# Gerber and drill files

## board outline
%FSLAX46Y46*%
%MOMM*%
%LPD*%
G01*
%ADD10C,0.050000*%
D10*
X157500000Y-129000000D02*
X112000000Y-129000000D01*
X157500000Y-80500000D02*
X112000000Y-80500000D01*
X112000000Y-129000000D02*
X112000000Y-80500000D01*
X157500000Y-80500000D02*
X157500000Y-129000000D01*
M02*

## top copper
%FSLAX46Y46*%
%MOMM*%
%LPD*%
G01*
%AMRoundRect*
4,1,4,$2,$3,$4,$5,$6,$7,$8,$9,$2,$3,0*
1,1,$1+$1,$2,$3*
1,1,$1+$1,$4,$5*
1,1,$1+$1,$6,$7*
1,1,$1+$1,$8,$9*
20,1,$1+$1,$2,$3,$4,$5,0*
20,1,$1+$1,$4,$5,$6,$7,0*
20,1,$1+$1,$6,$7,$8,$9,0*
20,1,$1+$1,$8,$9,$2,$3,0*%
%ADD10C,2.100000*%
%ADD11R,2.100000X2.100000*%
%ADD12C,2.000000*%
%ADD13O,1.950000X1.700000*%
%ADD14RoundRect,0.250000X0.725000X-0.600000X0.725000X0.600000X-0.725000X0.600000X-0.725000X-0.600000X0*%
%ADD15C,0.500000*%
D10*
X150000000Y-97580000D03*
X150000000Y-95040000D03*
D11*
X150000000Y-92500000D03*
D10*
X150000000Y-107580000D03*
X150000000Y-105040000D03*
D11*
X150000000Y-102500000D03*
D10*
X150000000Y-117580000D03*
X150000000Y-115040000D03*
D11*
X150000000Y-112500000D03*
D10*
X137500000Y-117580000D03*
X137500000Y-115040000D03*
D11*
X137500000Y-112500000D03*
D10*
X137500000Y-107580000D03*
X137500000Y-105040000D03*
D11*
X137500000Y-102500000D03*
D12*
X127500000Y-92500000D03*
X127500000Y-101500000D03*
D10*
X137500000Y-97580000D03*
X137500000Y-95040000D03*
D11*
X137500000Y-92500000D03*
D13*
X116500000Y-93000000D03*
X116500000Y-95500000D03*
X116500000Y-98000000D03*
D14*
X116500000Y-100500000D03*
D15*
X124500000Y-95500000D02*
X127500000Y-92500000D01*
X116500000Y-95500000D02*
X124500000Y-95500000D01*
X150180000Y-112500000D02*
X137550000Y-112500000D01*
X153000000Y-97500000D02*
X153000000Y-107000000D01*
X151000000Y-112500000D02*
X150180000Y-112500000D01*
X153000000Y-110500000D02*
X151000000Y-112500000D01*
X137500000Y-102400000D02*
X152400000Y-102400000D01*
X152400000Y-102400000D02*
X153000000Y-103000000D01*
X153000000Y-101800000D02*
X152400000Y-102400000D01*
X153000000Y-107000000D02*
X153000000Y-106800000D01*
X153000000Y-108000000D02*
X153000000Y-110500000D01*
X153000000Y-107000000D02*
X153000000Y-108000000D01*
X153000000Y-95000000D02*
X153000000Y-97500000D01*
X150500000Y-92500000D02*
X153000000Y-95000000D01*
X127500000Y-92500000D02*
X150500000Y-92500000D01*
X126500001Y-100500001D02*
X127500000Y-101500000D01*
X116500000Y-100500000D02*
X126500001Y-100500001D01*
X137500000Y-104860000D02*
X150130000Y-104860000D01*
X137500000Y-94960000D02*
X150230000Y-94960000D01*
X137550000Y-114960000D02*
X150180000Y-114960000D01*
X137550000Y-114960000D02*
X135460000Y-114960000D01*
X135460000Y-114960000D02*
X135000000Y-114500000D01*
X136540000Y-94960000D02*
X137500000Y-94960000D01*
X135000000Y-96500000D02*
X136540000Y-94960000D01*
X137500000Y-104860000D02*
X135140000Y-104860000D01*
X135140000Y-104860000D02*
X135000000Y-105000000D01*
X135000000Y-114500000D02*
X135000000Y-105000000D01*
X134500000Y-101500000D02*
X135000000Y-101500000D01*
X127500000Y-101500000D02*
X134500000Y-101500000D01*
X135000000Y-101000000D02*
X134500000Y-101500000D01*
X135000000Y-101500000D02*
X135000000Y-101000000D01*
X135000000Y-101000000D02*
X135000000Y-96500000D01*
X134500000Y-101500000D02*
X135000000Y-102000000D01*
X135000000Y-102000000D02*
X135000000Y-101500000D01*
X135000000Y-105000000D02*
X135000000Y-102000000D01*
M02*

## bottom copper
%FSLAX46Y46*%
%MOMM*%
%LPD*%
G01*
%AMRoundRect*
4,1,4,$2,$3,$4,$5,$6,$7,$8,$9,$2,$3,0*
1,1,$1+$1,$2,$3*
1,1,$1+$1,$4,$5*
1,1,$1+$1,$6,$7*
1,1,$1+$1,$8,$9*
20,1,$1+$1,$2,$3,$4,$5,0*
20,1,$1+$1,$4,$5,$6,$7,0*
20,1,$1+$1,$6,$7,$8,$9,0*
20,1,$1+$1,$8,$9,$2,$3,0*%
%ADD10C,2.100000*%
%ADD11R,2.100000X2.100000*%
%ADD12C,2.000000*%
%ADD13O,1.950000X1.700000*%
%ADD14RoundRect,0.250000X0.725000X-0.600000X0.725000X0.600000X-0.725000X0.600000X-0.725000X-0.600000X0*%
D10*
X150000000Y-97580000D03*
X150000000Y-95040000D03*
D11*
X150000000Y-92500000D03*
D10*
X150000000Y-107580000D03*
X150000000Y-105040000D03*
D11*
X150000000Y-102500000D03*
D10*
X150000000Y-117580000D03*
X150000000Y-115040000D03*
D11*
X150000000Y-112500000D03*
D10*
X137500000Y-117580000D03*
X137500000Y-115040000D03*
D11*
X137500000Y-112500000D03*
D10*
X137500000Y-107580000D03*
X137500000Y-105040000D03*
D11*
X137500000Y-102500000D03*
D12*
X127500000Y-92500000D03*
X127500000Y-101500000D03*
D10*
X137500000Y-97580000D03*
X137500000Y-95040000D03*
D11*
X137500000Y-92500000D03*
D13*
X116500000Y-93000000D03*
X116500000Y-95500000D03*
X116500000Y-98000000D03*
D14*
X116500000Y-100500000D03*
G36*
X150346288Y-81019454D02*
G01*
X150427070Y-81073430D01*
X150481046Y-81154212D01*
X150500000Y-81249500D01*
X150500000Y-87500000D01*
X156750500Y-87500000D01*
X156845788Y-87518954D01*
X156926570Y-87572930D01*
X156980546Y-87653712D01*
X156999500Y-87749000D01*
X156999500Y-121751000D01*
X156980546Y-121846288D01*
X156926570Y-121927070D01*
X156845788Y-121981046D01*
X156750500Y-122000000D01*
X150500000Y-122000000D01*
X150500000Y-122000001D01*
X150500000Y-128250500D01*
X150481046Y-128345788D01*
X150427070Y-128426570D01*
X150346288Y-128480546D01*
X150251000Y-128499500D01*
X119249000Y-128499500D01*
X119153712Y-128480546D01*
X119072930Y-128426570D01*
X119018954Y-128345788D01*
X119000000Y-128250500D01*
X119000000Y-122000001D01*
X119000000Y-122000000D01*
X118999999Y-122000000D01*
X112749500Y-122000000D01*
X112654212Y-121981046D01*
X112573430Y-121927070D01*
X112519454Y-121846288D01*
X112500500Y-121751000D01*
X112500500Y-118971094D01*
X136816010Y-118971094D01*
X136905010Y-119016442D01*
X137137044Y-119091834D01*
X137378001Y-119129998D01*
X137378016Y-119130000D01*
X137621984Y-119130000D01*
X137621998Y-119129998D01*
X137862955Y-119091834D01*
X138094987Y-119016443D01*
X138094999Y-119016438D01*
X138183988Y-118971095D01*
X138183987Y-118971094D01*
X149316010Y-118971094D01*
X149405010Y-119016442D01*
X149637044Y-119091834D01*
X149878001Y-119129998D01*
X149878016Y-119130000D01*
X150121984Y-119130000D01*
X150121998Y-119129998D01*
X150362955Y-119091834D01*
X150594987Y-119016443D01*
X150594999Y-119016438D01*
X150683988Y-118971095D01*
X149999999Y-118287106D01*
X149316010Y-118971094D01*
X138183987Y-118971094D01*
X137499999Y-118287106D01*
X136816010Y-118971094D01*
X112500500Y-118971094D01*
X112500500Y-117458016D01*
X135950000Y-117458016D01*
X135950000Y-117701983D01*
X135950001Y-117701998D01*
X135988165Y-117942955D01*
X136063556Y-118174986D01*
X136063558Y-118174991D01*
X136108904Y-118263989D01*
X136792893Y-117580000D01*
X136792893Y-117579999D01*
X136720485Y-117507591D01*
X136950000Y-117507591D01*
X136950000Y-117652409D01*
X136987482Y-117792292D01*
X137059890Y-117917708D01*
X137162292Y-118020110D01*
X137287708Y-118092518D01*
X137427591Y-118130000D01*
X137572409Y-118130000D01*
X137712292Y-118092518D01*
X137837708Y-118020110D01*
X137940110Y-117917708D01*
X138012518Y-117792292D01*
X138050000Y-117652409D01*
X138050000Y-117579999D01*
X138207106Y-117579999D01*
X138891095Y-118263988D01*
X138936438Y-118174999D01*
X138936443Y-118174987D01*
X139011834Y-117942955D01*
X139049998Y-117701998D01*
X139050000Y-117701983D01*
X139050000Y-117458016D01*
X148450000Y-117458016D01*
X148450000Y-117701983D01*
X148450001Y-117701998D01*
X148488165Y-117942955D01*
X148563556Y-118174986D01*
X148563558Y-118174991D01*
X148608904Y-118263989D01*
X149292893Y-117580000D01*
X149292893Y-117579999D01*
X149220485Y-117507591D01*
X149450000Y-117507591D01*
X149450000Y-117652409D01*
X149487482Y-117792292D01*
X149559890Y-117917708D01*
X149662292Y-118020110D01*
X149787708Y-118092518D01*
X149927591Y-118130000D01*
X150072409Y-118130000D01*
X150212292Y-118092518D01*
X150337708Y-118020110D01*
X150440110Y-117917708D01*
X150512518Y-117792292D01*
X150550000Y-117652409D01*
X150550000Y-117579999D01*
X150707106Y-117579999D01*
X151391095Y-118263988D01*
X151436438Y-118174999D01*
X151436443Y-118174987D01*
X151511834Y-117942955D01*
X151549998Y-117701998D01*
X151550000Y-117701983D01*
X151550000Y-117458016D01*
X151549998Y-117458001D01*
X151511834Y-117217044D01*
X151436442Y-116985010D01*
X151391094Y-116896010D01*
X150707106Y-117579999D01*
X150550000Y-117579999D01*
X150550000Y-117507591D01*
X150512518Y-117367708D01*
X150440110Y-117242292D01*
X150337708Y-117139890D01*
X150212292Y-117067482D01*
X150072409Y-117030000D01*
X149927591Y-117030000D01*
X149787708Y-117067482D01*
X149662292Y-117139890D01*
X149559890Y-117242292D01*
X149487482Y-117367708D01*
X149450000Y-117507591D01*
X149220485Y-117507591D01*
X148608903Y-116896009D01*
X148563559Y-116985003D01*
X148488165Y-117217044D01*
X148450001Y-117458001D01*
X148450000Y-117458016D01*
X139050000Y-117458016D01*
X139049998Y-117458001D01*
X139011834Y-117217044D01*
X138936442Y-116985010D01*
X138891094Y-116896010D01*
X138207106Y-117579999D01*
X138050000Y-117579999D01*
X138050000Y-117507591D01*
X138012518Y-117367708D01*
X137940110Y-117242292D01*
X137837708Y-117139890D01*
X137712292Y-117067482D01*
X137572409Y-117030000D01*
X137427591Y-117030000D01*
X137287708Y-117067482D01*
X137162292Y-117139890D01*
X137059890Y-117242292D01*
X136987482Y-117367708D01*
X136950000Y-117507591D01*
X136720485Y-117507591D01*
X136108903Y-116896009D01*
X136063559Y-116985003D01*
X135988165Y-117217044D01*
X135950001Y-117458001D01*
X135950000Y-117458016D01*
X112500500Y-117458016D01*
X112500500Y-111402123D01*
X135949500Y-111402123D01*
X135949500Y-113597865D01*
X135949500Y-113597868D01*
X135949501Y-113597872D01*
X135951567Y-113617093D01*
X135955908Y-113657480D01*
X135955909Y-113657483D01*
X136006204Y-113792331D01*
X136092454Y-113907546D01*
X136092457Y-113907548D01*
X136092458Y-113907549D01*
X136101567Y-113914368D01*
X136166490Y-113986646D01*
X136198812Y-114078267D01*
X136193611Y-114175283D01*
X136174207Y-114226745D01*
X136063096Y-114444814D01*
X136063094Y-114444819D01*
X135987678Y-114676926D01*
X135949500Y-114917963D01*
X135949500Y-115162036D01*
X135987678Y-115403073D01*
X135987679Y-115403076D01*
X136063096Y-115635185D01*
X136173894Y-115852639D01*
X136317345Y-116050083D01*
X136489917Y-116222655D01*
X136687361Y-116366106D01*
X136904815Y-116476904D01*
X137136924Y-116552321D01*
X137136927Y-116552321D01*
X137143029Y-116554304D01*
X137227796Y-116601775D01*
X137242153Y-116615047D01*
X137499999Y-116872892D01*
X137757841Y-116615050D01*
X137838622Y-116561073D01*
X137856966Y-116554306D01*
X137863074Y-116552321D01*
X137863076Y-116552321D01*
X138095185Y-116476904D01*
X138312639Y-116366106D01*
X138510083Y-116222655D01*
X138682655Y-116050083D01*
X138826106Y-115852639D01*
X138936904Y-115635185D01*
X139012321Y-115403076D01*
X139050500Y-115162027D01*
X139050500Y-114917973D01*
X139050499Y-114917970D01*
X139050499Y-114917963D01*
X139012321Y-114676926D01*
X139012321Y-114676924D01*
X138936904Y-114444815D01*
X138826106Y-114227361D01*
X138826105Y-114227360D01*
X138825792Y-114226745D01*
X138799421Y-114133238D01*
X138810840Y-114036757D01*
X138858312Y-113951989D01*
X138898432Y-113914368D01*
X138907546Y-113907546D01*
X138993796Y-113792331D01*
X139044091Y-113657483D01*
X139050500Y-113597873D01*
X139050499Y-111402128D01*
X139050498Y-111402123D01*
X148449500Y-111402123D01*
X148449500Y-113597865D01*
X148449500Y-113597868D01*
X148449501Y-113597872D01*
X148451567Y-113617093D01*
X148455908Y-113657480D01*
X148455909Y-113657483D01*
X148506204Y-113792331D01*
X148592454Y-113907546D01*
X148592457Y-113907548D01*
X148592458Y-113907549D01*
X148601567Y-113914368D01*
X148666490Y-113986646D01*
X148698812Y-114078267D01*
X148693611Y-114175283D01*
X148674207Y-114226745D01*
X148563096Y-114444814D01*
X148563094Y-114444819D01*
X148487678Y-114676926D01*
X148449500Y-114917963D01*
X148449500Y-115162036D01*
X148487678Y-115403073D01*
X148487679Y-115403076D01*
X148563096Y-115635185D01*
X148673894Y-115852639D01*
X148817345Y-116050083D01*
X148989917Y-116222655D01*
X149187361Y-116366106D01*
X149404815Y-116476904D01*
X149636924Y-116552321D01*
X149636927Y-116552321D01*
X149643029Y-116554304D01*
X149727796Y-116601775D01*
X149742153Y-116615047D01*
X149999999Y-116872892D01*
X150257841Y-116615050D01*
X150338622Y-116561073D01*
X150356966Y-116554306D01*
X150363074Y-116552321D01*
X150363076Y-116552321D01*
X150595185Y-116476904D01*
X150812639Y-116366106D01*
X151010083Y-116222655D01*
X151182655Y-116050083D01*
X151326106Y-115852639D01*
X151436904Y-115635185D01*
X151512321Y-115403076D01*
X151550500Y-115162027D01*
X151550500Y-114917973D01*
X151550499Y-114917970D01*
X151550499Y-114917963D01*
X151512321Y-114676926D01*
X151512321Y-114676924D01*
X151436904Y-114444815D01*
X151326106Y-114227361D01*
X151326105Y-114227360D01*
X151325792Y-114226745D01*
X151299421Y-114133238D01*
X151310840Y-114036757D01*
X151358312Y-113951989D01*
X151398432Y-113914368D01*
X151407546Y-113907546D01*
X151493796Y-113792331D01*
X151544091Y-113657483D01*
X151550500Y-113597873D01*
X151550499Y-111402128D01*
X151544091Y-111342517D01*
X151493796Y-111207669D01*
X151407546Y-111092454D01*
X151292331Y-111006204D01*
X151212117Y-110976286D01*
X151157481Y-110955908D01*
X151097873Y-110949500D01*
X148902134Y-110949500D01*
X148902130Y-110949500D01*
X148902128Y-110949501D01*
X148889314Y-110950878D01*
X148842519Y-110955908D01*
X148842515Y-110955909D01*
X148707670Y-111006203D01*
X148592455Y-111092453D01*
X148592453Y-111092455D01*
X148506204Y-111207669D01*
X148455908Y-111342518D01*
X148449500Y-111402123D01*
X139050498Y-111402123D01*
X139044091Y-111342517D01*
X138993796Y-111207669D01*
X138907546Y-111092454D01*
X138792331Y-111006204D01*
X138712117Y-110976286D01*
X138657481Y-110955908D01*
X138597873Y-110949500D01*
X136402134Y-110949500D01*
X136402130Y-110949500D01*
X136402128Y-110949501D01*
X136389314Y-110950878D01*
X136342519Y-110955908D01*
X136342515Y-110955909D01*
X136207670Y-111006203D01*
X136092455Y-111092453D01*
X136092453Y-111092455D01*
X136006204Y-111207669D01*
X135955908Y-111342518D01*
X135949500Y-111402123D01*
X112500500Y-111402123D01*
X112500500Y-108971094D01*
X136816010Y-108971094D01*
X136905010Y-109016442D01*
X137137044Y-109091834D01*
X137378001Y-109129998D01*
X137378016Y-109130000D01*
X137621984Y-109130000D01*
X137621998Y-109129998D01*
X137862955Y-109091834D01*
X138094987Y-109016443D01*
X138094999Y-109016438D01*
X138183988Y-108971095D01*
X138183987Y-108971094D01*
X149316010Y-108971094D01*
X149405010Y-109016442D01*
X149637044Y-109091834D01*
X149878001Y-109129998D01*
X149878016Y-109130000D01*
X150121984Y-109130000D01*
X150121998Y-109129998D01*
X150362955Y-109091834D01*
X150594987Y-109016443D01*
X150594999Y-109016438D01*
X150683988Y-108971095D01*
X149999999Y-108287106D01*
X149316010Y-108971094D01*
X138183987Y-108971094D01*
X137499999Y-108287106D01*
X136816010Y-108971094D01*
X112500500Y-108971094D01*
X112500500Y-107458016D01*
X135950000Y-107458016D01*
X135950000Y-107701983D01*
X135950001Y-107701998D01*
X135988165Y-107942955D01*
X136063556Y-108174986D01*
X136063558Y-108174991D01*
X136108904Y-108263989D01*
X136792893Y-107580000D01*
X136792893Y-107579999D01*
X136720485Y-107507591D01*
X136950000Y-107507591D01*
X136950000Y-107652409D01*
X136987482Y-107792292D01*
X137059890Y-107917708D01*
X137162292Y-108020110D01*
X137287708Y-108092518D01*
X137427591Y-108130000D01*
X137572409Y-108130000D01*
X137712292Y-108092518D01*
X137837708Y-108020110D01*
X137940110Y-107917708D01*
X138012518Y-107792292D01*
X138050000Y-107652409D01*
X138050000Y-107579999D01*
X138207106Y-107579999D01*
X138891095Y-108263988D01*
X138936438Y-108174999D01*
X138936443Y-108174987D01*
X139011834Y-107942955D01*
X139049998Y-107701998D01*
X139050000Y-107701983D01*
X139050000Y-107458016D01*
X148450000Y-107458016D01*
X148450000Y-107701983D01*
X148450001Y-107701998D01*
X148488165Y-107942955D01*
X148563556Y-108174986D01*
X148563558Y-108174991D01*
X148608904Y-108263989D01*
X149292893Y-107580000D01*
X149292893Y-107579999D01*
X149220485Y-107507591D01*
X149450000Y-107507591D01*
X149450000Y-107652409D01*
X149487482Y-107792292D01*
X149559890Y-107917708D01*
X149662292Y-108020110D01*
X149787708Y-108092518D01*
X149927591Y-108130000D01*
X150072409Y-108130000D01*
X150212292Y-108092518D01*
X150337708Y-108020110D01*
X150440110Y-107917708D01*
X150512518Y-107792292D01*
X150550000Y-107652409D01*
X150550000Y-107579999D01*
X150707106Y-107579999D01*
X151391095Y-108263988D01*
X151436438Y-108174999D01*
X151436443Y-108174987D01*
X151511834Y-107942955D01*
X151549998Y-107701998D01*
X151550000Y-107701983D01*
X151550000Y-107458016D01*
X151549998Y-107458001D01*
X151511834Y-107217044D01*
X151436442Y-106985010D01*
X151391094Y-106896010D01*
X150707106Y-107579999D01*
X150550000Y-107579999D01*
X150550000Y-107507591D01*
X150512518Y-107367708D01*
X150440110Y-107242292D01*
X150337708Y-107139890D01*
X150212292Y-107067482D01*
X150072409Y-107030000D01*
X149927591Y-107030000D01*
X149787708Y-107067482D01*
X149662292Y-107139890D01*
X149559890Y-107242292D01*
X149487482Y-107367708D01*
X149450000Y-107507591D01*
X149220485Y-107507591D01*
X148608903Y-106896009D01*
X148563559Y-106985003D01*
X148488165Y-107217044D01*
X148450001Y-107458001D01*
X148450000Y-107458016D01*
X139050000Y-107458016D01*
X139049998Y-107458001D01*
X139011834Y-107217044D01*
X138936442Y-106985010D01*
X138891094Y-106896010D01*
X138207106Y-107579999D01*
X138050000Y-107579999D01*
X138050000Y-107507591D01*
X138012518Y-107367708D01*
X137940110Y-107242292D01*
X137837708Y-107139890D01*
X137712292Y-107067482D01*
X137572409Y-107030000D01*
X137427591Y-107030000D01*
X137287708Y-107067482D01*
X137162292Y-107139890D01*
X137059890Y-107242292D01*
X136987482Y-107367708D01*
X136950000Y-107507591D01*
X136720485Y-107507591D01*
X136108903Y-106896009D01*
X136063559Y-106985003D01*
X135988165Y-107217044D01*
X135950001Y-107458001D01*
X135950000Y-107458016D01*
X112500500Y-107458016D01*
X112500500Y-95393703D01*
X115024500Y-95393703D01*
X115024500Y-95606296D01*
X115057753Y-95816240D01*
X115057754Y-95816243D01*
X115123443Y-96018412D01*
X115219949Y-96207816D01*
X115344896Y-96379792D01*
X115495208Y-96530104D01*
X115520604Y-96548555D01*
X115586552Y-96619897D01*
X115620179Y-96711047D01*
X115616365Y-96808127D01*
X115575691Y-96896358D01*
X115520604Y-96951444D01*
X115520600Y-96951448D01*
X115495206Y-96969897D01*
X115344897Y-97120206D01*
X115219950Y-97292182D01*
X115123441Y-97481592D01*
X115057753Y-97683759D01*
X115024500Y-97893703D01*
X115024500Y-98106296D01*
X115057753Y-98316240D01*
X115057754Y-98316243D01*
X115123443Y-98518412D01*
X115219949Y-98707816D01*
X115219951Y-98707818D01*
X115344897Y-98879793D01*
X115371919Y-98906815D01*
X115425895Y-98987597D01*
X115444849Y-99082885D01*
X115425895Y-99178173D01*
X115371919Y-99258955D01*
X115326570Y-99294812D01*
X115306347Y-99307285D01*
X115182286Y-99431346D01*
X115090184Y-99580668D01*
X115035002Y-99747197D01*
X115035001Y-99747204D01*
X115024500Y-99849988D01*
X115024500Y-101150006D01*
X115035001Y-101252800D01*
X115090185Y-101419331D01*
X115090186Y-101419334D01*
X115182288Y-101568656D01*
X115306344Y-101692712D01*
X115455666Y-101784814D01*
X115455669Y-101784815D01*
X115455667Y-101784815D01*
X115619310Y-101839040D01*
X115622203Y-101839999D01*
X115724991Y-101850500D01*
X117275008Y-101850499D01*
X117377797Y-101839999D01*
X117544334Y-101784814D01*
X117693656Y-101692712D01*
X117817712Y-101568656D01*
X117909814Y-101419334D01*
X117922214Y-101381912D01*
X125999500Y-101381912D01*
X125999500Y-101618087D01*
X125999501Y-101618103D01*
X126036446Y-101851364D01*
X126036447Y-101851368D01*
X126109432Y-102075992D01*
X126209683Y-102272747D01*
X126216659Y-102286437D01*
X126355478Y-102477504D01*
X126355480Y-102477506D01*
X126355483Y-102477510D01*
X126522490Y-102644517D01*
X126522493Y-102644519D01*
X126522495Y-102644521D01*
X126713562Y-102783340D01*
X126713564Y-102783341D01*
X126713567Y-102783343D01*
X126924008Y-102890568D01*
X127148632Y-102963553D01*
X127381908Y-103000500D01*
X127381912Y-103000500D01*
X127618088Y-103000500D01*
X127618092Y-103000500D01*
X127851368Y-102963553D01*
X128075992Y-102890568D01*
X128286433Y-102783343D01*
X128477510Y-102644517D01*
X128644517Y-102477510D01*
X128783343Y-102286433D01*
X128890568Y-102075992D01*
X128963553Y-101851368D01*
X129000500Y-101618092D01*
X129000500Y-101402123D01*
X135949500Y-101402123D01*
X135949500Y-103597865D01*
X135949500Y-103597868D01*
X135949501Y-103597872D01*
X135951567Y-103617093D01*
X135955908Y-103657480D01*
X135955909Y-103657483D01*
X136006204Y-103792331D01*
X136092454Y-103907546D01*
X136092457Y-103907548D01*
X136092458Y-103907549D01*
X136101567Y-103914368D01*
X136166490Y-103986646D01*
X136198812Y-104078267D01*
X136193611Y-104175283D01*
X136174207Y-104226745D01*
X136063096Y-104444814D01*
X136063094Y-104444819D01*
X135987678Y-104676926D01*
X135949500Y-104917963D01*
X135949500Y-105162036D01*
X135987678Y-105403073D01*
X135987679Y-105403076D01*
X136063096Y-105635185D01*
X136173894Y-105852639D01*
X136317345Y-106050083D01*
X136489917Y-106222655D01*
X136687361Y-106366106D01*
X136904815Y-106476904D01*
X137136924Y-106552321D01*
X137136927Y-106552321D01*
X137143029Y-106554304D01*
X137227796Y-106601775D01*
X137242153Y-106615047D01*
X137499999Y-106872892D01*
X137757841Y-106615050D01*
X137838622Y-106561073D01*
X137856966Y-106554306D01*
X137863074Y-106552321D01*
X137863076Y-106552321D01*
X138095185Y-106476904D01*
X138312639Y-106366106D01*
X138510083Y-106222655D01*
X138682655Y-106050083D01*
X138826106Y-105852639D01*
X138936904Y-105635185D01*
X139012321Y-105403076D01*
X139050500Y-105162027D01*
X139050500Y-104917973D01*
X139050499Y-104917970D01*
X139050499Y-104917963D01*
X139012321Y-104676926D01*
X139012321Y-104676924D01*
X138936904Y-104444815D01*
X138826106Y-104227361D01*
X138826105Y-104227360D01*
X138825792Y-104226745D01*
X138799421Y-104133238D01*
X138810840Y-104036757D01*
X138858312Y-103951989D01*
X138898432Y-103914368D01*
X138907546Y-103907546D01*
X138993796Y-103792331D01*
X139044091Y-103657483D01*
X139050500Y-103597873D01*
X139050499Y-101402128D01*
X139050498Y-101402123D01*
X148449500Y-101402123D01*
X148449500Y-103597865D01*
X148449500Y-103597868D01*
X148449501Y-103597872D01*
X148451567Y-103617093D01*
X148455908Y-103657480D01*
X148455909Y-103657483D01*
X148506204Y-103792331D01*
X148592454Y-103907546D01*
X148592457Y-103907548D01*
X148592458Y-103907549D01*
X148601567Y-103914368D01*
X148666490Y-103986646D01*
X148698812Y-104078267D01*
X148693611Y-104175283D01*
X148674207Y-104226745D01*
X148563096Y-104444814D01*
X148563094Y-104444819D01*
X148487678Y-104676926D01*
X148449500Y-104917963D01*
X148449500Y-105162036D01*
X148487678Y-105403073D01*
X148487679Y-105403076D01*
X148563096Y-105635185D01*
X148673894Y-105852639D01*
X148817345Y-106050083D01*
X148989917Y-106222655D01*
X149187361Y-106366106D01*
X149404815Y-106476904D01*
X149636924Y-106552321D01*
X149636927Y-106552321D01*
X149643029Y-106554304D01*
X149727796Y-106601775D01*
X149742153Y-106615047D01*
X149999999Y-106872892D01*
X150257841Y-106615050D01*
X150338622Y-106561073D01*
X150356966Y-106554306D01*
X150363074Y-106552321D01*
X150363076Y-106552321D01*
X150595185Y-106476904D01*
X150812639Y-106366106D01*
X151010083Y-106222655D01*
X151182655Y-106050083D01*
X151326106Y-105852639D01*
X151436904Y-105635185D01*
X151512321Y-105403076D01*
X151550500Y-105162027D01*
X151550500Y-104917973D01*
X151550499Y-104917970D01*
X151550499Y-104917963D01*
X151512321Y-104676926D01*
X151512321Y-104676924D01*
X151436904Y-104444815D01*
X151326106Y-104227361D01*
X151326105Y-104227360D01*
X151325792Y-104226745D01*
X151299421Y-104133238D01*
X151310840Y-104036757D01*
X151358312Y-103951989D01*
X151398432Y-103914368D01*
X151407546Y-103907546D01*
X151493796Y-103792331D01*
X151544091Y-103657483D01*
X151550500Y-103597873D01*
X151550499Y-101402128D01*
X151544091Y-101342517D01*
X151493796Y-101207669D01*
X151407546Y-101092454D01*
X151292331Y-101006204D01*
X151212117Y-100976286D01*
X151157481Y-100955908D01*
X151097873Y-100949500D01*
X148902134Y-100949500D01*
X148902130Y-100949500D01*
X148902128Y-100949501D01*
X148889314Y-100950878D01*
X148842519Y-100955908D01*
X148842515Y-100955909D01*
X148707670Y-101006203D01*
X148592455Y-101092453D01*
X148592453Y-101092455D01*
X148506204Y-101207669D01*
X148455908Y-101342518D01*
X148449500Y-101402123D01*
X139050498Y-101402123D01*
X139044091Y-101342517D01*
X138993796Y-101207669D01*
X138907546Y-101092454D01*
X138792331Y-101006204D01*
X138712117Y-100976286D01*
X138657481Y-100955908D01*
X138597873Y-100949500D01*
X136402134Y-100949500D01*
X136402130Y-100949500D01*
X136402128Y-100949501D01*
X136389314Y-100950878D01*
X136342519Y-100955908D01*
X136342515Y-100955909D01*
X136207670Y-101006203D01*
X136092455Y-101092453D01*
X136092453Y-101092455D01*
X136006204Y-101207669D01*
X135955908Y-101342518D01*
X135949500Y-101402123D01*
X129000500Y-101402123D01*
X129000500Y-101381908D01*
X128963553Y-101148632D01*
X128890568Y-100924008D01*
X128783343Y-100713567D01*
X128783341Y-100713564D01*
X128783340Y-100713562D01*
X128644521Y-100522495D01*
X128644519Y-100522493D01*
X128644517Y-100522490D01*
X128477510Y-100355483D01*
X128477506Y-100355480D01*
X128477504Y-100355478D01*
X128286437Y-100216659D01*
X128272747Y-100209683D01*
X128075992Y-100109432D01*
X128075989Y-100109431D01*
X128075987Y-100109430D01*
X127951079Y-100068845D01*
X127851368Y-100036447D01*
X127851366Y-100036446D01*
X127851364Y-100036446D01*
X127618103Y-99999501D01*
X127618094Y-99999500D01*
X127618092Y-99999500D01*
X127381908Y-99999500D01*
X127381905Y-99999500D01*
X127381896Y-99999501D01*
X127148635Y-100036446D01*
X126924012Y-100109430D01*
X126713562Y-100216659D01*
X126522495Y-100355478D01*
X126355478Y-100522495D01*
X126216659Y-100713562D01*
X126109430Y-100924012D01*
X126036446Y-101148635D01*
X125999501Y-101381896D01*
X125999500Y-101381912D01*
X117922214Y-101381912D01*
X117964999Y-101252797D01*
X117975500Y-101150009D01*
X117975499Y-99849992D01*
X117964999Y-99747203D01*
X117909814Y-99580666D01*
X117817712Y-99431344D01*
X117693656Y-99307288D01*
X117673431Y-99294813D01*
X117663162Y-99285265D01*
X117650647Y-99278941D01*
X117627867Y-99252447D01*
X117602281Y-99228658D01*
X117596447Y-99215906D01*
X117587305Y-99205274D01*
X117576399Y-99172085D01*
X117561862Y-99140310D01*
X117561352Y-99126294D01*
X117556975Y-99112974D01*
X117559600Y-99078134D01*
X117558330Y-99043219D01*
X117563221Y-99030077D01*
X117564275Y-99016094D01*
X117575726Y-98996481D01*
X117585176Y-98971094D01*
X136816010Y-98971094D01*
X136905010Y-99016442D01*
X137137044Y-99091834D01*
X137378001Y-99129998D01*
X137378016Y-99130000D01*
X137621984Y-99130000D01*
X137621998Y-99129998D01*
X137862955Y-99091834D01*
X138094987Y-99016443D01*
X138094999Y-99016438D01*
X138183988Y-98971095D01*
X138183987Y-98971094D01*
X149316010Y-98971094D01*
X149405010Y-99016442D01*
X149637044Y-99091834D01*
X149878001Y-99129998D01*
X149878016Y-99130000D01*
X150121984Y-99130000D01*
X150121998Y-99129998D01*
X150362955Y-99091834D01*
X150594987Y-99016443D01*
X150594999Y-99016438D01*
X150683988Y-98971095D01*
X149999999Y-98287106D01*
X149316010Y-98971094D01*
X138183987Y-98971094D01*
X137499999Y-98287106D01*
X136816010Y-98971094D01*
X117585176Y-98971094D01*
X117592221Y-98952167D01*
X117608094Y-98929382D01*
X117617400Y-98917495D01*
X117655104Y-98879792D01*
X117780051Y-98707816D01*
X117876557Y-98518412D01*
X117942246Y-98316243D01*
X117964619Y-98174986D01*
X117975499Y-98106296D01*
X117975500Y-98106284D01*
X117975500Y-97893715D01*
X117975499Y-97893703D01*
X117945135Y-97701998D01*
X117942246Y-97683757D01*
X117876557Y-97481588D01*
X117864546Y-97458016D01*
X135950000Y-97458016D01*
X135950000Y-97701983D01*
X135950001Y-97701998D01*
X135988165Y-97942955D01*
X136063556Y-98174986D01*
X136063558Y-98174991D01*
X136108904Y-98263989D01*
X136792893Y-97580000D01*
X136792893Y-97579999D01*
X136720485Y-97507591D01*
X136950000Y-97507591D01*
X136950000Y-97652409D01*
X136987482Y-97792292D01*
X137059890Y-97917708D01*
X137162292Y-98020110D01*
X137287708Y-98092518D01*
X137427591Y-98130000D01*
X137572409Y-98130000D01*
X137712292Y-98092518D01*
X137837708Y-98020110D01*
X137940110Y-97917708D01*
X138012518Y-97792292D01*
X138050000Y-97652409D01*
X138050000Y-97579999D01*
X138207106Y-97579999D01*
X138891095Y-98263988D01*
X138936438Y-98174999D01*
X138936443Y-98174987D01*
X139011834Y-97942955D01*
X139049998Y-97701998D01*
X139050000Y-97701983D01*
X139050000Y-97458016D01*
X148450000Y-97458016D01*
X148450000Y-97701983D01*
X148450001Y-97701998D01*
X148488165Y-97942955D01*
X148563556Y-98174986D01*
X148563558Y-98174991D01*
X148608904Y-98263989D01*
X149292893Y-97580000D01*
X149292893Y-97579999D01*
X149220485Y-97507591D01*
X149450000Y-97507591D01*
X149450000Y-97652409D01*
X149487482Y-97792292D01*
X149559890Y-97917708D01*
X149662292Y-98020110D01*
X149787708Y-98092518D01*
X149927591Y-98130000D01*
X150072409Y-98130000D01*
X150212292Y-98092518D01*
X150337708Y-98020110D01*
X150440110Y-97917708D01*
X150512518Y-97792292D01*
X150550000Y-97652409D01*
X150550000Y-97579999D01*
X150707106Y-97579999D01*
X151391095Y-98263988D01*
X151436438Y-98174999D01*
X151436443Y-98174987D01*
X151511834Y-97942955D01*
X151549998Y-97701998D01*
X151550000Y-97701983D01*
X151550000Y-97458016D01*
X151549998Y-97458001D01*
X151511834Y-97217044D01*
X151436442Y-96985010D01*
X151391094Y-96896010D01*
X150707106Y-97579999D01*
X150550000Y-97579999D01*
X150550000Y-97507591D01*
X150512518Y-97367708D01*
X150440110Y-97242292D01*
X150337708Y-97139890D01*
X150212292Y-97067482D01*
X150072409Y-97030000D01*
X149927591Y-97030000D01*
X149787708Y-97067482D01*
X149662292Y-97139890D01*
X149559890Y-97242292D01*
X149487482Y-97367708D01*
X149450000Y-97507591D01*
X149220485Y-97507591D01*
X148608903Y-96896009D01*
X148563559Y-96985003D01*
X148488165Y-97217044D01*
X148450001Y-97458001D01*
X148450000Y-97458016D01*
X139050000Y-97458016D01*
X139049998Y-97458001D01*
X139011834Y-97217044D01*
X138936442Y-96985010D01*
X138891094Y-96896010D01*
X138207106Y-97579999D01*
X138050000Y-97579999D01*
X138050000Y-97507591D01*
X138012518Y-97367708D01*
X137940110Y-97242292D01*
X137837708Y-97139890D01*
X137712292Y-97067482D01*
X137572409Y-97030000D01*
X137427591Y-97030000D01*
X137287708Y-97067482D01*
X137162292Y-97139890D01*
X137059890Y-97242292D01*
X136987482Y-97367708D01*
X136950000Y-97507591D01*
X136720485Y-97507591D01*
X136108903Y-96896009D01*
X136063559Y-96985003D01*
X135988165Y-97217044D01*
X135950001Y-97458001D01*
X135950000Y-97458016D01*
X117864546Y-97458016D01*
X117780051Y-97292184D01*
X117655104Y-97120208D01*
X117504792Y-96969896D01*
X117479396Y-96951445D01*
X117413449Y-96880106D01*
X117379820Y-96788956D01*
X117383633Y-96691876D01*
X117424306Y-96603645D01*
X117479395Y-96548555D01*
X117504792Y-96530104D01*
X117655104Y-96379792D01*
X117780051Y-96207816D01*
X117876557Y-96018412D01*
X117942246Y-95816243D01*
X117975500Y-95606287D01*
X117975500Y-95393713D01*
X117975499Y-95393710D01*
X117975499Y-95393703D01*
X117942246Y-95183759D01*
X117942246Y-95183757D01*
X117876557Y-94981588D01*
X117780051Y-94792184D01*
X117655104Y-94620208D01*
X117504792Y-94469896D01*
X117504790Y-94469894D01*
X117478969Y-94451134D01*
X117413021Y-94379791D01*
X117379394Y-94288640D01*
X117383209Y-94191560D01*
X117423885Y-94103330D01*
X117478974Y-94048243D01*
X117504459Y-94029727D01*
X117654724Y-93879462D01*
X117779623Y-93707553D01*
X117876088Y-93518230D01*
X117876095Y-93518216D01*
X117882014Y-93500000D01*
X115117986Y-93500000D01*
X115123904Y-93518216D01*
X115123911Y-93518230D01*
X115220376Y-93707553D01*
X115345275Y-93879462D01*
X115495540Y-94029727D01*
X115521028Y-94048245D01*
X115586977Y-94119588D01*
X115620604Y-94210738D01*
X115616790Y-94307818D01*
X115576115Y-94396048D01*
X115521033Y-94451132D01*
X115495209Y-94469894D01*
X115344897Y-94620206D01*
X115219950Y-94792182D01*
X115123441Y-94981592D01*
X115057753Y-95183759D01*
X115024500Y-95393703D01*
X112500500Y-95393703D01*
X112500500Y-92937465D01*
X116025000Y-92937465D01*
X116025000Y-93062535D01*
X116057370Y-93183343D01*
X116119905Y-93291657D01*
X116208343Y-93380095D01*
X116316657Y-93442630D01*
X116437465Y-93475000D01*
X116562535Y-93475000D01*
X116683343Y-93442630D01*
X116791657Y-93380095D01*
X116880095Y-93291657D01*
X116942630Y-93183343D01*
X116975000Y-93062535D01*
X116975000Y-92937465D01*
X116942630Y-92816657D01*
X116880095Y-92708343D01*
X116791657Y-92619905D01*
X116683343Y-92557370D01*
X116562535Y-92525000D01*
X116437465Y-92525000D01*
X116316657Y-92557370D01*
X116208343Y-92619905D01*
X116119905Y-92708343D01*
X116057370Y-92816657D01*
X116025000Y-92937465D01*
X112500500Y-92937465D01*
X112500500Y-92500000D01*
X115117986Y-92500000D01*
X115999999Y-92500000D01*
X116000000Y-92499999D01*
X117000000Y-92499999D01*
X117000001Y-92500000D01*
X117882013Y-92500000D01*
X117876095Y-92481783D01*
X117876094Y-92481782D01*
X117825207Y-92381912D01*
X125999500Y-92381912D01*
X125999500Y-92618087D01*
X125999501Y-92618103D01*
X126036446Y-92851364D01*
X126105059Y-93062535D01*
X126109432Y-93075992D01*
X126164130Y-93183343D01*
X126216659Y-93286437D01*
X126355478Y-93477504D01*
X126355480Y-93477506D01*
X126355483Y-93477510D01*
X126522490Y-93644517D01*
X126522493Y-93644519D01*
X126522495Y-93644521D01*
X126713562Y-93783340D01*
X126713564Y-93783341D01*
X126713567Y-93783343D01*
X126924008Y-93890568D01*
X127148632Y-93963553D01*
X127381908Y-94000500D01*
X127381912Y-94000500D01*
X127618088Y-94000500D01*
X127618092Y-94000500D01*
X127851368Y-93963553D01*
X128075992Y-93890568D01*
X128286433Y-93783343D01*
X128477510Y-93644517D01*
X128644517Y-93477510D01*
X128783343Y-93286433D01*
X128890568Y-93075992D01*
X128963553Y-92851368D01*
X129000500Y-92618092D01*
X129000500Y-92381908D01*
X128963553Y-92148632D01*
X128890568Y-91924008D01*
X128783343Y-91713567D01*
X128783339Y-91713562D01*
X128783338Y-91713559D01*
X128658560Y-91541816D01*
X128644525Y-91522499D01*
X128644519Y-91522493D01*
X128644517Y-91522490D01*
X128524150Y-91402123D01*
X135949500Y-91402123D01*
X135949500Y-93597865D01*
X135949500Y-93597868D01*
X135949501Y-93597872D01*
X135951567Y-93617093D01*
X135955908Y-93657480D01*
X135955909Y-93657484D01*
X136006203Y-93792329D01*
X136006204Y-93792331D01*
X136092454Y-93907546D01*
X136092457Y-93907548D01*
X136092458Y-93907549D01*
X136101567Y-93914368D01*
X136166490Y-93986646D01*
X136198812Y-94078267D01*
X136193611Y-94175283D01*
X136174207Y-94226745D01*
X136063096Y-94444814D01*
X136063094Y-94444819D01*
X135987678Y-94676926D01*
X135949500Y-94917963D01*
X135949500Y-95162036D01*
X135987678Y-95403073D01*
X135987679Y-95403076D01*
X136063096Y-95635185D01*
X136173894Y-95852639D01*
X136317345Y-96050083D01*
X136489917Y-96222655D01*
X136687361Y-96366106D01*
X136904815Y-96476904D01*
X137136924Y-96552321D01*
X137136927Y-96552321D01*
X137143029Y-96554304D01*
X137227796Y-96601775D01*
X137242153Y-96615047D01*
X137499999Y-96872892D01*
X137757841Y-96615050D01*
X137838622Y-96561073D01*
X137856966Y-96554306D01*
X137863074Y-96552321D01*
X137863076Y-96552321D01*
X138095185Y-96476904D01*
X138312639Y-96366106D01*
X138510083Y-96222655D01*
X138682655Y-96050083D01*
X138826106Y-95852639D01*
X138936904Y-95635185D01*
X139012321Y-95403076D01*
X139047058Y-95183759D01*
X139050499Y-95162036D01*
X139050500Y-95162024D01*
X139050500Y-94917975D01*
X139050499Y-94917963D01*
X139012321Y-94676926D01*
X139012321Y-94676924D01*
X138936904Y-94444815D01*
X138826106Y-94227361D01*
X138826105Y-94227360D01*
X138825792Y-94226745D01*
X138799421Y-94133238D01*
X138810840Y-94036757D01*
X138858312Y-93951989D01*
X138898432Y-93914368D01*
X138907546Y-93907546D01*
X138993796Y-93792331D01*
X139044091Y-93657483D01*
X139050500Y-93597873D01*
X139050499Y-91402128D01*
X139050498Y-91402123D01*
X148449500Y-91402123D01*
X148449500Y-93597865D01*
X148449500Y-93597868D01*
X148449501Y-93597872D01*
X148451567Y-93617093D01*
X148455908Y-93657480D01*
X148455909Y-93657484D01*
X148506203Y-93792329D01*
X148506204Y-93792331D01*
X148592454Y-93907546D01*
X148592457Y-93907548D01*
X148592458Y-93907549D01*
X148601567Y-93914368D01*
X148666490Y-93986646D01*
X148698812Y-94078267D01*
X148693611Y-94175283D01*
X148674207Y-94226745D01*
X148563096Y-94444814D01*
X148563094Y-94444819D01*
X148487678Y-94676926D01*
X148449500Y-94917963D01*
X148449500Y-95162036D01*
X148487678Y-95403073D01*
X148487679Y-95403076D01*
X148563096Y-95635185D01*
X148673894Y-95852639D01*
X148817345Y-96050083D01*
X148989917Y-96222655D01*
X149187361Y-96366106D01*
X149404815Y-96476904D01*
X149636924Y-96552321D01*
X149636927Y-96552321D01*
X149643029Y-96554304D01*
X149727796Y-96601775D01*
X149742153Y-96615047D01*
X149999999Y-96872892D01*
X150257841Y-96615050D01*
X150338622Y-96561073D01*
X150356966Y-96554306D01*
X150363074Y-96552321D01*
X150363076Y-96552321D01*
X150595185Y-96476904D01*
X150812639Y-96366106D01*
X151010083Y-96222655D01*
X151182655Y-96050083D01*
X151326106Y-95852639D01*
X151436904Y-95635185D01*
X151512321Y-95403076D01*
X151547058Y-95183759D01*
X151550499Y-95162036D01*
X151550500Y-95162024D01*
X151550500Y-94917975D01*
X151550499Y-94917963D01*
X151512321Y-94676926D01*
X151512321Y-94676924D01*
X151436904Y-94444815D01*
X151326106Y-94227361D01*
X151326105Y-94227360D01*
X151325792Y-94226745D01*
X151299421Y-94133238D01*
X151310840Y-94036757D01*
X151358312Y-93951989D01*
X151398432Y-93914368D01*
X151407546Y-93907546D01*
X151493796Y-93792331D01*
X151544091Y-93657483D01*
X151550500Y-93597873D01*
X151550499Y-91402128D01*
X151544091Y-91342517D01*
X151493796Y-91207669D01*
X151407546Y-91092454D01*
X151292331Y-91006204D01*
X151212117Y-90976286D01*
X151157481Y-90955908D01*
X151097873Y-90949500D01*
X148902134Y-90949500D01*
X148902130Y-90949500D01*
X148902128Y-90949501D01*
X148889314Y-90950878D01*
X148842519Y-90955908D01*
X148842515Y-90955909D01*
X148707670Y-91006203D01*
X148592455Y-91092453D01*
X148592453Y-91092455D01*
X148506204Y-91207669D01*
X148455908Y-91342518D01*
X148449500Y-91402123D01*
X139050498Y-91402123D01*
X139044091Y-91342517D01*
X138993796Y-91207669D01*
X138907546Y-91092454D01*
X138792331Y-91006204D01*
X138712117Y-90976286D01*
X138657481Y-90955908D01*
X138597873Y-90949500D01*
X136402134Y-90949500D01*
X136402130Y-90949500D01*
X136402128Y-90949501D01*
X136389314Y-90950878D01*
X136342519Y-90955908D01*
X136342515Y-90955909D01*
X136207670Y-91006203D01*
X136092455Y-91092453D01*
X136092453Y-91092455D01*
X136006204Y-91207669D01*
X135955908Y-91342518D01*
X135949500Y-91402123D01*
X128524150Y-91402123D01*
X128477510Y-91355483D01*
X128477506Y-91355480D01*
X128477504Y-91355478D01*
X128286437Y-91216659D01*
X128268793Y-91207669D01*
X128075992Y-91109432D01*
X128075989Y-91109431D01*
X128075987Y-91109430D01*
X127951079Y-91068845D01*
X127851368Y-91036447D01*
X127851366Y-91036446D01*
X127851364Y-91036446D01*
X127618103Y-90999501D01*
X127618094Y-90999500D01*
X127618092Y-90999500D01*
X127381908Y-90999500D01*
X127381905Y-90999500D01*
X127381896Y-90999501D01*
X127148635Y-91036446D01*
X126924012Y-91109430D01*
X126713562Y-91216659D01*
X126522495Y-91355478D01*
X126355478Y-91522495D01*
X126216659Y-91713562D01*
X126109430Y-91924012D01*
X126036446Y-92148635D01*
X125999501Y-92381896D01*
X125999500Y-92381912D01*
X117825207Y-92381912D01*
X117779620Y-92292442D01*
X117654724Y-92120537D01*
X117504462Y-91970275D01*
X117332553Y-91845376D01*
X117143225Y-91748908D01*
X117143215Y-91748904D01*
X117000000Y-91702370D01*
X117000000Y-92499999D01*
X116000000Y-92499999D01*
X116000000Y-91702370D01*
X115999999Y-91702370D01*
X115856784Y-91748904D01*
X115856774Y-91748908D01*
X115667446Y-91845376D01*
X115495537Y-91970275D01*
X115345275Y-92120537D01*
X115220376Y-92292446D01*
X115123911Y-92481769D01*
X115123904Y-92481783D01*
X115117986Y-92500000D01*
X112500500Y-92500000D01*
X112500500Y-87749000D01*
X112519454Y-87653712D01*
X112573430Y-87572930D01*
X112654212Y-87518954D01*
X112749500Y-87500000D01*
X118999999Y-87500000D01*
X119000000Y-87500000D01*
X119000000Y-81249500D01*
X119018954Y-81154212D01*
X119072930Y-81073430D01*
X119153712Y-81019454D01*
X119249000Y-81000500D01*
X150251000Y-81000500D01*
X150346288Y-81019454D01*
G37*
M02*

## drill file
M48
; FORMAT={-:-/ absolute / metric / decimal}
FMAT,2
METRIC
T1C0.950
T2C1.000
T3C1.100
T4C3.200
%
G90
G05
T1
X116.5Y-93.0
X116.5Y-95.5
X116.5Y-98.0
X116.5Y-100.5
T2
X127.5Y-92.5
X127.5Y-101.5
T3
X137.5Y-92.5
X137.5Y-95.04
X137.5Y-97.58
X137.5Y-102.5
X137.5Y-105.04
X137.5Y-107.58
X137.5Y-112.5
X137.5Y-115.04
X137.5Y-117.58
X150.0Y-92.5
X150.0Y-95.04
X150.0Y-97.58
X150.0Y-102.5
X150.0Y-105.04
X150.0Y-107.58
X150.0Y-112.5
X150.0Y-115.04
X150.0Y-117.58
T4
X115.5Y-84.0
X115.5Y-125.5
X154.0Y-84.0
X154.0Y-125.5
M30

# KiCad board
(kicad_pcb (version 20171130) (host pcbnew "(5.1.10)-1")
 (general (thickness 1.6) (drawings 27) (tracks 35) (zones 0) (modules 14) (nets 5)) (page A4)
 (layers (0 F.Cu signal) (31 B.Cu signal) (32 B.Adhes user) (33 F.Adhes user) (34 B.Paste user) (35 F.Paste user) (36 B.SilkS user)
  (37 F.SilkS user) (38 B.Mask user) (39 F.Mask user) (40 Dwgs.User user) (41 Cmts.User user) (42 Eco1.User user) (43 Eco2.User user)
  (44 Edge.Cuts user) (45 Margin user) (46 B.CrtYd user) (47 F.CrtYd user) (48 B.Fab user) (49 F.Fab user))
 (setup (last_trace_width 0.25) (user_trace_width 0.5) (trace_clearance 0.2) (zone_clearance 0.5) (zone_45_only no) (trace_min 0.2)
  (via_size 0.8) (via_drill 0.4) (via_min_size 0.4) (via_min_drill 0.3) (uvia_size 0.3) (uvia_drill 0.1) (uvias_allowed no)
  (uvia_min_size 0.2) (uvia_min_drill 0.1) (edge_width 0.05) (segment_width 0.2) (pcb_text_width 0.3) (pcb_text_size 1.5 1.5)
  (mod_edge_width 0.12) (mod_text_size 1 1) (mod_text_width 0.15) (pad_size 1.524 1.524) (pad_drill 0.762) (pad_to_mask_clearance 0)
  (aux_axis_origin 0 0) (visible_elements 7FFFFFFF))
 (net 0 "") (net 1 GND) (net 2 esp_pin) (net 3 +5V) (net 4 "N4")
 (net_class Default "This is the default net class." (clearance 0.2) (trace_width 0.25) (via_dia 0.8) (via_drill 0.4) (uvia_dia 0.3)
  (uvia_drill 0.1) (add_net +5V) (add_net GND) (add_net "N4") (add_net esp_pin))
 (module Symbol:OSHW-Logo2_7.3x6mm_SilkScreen (layer F.Cu) (at 137.5 124.5)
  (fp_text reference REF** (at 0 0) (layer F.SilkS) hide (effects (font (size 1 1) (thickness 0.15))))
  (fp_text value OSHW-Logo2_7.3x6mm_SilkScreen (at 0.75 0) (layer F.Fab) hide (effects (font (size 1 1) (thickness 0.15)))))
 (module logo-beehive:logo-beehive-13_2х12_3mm (layer F.Cu) (at 123 109.22)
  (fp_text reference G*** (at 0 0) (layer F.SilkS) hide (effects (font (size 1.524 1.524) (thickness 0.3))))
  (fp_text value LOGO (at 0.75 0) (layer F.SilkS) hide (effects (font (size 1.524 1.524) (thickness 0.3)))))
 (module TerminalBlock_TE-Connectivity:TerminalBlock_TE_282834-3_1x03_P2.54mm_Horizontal (layer F.Cu) (at 150 92.5 270)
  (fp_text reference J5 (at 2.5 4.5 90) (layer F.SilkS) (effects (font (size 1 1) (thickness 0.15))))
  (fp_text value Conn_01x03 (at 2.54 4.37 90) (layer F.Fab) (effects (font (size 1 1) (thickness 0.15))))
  (pad 3 thru_hole circle (at 5.08 0 270) (size 2.1 2.1) (drill 1.1) (layers *.Cu *.Mask) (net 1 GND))
  (pad 2 thru_hole circle (at 2.54 0 270) (size 2.1 2.1) (drill 1.1) (layers *.Cu *.Mask) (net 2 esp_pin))
  (pad 1 thru_hole rect (at 0 0 270) (size 2.1 2.1) (drill 1.1) (layers *.Cu *.Mask) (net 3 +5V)))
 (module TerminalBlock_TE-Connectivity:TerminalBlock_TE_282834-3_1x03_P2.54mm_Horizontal (layer F.Cu) (at 150 102.5 270)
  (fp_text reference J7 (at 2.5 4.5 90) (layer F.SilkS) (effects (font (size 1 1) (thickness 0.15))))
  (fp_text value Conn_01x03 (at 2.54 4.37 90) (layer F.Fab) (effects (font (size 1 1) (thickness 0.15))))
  (pad 3 thru_hole circle (at 5.08 0 270) (size 2.1 2.1) (drill 1.1) (layers *.Cu *.Mask) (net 1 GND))
  (pad 2 thru_hole circle (at 2.54 0 270) (size 2.1 2.1) (drill 1.1) (layers *.Cu *.Mask) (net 2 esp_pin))
  (pad 1 thru_hole rect (at 0 0 270) (size 2.1 2.1) (drill 1.1) (layers *.Cu *.Mask) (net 3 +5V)))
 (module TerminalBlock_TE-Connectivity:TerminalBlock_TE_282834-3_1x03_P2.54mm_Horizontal (layer F.Cu) (at 150 112.5 270)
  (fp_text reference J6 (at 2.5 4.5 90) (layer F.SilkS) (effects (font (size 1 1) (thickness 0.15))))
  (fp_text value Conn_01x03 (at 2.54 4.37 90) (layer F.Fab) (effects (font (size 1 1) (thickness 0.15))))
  (pad 3 thru_hole circle (at 5.08 0 270) (size 2.1 2.1) (drill 1.1) (layers *.Cu *.Mask) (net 1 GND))
  (pad 2 thru_hole circle (at 2.54 0 270) (size 2.1 2.1) (drill 1.1) (layers *.Cu *.Mask) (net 2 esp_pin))
  (pad 1 thru_hole rect (at 0 0 270) (size 2.1 2.1) (drill 1.1) (layers *.Cu *.Mask) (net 3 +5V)))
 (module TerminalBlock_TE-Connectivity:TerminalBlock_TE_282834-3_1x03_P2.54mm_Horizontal (layer F.Cu) (at 137.5 112.5 270)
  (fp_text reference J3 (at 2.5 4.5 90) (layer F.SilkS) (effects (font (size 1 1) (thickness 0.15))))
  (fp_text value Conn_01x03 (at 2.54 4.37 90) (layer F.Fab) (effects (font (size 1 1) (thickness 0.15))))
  (pad 3 thru_hole circle (at 5.08 0 270) (size 2.1 2.1) (drill 1.1) (layers *.Cu *.Mask) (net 1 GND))
  (pad 2 thru_hole circle (at 2.54 0 270) (size 2.1 2.1) (drill 1.1) (layers *.Cu *.Mask) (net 2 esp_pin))
  (pad 1 thru_hole rect (at 0 0 270) (size 2.1 2.1) (drill 1.1) (layers *.Cu *.Mask) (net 3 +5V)))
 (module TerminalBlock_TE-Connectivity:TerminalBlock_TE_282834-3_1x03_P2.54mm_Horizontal (layer F.Cu) (at 137.5 102.5 270)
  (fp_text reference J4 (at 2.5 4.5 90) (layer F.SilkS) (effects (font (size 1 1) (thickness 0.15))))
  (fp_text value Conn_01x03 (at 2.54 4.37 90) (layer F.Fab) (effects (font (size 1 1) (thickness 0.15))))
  (pad 3 thru_hole circle (at 5.08 0 270) (size 2.1 2.1) (drill 1.1) (layers *.Cu *.Mask) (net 1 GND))
  (pad 2 thru_hole circle (at 2.54 0 270) (size 2.1 2.1) (drill 1.1) (layers *.Cu *.Mask) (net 2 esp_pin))
  (pad 1 thru_hole rect (at 0 0 270) (size 2.1 2.1) (drill 1.1) (layers *.Cu *.Mask) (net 3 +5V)))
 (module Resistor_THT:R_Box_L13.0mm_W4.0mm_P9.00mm (layer F.Cu) (at 127.5 101.5 90)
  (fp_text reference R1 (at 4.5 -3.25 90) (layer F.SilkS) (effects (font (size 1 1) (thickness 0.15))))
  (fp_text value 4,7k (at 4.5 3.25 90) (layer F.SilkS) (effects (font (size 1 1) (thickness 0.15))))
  (pad 2 thru_hole circle (at 9 0 90) (size 2 2) (drill 1) (layers *.Cu *.Mask) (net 3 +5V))
  (pad 1 thru_hole circle (at 0 0 90) (size 2 2) (drill 1) (layers *.Cu *.Mask) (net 2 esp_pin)))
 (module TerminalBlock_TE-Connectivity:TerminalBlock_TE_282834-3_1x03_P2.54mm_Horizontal (layer F.Cu) (at 137.5 92.5 270)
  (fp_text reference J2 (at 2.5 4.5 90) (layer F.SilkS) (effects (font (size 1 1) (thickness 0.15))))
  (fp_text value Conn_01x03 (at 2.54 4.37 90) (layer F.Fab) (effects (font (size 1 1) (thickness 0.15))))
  (pad 3 thru_hole circle (at 5.08 0 270) (size 2.1 2.1) (drill 1.1) (layers *.Cu *.Mask) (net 1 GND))
  (pad 2 thru_hole circle (at 2.54 0 270) (size 2.1 2.1) (drill 1.1) (layers *.Cu *.Mask) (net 2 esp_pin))
  (pad 1 thru_hole rect (at 0 0 270) (size 2.1 2.1) (drill 1.1) (layers *.Cu *.Mask) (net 3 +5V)))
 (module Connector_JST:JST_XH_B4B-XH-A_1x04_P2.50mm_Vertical (layer F.Cu) (at 116.5 100.5 90)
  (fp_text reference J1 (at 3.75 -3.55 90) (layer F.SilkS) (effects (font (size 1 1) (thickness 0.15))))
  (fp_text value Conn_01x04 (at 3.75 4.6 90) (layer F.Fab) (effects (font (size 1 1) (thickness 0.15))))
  (pad 4 thru_hole oval (at 7.5 0 90) (size 1.7 1.95) (drill 0.95) (layers *.Cu *.Mask) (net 1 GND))
  (pad 3 thru_hole oval (at 5 0 90) (size 1.7 1.95) (drill 0.95) (layers *.Cu *.Mask) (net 3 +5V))
  (pad 2 thru_hole oval (at 2.5 0 90) (size 1.7 1.95) (drill 0.95) (layers *.Cu *.Mask) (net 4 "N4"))
  (pad 1 thru_hole roundrect (at 0 0 90) (size 1.7 1.95) (drill 0.95) (layers *.Cu *.Mask) (roundrect_rratio 0.1470588235294118)
   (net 2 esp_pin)))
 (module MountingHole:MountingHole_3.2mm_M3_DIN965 (layer F.Cu) (at 154 125.5)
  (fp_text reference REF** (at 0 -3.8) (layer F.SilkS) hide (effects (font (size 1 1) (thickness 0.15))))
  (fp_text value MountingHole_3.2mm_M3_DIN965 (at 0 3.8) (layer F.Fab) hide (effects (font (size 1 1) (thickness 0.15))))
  (pad 1 np_thru_hole circle (at 0 0) (size 3.2 3.2) (drill 3.2) (layers *.Cu *.Mask)))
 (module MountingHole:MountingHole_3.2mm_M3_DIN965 (layer F.Cu) (at 154 84)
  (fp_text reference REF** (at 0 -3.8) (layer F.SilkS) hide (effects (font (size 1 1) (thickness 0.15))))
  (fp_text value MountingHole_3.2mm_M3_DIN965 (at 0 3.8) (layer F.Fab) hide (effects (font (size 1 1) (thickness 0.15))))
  (pad 1 np_thru_hole circle (at 0 0) (size 3.2 3.2) (drill 3.2) (layers *.Cu *.Mask)))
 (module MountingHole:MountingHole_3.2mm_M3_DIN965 (layer F.Cu) (at 115.5 125.5)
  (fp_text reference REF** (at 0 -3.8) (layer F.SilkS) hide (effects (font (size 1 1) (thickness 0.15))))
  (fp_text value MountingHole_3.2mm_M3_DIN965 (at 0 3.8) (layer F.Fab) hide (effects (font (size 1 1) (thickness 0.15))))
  (pad 1 np_thru_hole circle (at 0 0) (size 3.2 3.2) (drill 3.2) (layers *.Cu *.Mask)))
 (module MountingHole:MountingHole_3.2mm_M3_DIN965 (layer F.Cu) (at 115.5 84)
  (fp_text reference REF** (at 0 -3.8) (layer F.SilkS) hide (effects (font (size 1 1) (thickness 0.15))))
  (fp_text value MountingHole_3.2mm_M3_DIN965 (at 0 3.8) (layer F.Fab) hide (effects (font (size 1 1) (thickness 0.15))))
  (pad 1 np_thru_hole circle (at 0 0) (size 3.2 3.2) (drill 3.2) (layers *.Cu *.Mask)))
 (gr_line (start 157.5 129) (end 112 129) (layer Edge.Cuts) (width 0.05))
 (gr_line (start 157.5 80.5) (end 112 80.5) (layer Edge.Cuts) (width 0.05))
 (gr_line (start 112 129) (end 112 80.5) (layer Edge.Cuts) (width 0.05))
 (gr_line (start 157.5 80.5) (end 157.5 129) (layer Edge.Cuts) (width 0.05))
 (segment (start 124.5 95.5) (end 127.5 92.5) (width 0.5) (layer F.Cu) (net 3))
 (segment (start 116.5 95.5) (end 124.5 95.5) (width 0.5) (layer F.Cu) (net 3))
 (segment (start 150.18 112.5) (end 137.55 112.5) (width 0.5) (layer F.Cu) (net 3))
 (segment (start 153 97.5) (end 153 107) (width 0.5) (layer F.Cu) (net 3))
 (segment (start 151 112.5) (end 150.18 112.5) (width 0.5) (layer F.Cu) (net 3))
 (segment (start 153 110.5) (end 151 112.5) (width 0.5) (layer F.Cu) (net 3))
 (segment (start 137.5 102.4) (end 152.4 102.4) (width 0.5) (layer F.Cu) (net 3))
 (segment (start 152.4 102.4) (end 153 103) (width 0.5) (layer F.Cu) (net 3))
 (segment (start 153 101.8) (end 152.4 102.4) (width 0.5) (layer F.Cu) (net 3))
 (segment (start 153 107) (end 153 106.8) (width 0.5) (layer F.Cu) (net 3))
 (segment (start 153 108) (end 153 110.5) (width 0.5) (layer F.Cu) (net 3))
 (segment (start 153 107) (end 153 108) (width 0.5) (layer F.Cu) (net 3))
 (segment (start 153 95) (end 153 97.5) (width 0.5) (layer F.Cu) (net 3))
 (segment (start 150.5 92.5) (end 153 95) (width 0.5) (layer F.Cu) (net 3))
 (segment (start 127.5 92.5) (end 150.5 92.5) (width 0.5) (layer F.Cu) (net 3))
 (segment (start 126.500001 100.500001) (end 127.5 101.5) (width 0.5) (layer F.Cu) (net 2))
 (segment (start 116.5 100.5) (end 126.500001 100.500001) (width 0.5) (layer F.Cu) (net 2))
 (segment (start 137.5 104.86) (end 150.13 104.86) (width 0.5) (layer F.Cu) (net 2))
 (segment (start 137.5 94.96) (end 150.23 94.96) (width 0.5) (layer F.Cu) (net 2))
 (segment (start 137.55 114.96) (end 150.18 114.96) (width 0.5) (layer F.Cu) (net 2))
 (segment (start 137.55 114.96) (end 135.46 114.96) (width 0.5) (layer F.Cu) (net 2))
 (segment (start 135.46 114.96) (end 135 114.5) (width 0.5) (layer F.Cu) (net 2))
 (segment (start 136.54 94.96) (end 137.5 94.96) (width 0.5) (layer F.Cu) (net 2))
 (segment (start 135 96.5) (end 136.54 94.96) (width 0.5) (layer F.Cu) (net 2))
 (segment (start 137.5 104.86) (end 135.14 104.86) (width 0.5) (layer F.Cu) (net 2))
 (segment (start 135.14 104.86) (end 135 105) (width 0.5) (layer F.Cu) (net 2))
 (segment (start 135 114.5) (end 135 105) (width 0.5) (layer F.Cu) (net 2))
 (segment (start 134.5 101.5) (end 135 101.5) (width 0.5) (layer F.Cu) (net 2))
 (segment (start 127.5 101.5) (end 134.5 101.5) (width 0.5) (layer F.Cu) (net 2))
 (segment (start 135 101) (end 134.5 101.5) (width 0.5) (layer F.Cu) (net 2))
 (segment (start 135 101.5) (end 135 101) (width 0.5) (layer F.Cu) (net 2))
 (segment (start 135 101) (end 135 96.5) (width 0.5) (layer F.Cu) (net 2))
 (segment (start 134.5 101.5) (end 135 102) (width 0.5) (layer F.Cu) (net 2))
 (segment (start 135 102) (end 135 101.5) (width 0.5) (layer F.Cu) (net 2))
 (segment (start 135 105) (end 135 102) (width 0.5) (layer F.Cu) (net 2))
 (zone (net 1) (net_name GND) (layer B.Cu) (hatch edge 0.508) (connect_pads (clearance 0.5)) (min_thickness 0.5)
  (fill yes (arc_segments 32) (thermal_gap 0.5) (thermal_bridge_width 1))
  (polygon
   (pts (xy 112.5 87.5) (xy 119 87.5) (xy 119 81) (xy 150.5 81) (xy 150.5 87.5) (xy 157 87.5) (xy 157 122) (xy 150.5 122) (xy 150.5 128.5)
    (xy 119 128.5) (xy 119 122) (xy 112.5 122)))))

